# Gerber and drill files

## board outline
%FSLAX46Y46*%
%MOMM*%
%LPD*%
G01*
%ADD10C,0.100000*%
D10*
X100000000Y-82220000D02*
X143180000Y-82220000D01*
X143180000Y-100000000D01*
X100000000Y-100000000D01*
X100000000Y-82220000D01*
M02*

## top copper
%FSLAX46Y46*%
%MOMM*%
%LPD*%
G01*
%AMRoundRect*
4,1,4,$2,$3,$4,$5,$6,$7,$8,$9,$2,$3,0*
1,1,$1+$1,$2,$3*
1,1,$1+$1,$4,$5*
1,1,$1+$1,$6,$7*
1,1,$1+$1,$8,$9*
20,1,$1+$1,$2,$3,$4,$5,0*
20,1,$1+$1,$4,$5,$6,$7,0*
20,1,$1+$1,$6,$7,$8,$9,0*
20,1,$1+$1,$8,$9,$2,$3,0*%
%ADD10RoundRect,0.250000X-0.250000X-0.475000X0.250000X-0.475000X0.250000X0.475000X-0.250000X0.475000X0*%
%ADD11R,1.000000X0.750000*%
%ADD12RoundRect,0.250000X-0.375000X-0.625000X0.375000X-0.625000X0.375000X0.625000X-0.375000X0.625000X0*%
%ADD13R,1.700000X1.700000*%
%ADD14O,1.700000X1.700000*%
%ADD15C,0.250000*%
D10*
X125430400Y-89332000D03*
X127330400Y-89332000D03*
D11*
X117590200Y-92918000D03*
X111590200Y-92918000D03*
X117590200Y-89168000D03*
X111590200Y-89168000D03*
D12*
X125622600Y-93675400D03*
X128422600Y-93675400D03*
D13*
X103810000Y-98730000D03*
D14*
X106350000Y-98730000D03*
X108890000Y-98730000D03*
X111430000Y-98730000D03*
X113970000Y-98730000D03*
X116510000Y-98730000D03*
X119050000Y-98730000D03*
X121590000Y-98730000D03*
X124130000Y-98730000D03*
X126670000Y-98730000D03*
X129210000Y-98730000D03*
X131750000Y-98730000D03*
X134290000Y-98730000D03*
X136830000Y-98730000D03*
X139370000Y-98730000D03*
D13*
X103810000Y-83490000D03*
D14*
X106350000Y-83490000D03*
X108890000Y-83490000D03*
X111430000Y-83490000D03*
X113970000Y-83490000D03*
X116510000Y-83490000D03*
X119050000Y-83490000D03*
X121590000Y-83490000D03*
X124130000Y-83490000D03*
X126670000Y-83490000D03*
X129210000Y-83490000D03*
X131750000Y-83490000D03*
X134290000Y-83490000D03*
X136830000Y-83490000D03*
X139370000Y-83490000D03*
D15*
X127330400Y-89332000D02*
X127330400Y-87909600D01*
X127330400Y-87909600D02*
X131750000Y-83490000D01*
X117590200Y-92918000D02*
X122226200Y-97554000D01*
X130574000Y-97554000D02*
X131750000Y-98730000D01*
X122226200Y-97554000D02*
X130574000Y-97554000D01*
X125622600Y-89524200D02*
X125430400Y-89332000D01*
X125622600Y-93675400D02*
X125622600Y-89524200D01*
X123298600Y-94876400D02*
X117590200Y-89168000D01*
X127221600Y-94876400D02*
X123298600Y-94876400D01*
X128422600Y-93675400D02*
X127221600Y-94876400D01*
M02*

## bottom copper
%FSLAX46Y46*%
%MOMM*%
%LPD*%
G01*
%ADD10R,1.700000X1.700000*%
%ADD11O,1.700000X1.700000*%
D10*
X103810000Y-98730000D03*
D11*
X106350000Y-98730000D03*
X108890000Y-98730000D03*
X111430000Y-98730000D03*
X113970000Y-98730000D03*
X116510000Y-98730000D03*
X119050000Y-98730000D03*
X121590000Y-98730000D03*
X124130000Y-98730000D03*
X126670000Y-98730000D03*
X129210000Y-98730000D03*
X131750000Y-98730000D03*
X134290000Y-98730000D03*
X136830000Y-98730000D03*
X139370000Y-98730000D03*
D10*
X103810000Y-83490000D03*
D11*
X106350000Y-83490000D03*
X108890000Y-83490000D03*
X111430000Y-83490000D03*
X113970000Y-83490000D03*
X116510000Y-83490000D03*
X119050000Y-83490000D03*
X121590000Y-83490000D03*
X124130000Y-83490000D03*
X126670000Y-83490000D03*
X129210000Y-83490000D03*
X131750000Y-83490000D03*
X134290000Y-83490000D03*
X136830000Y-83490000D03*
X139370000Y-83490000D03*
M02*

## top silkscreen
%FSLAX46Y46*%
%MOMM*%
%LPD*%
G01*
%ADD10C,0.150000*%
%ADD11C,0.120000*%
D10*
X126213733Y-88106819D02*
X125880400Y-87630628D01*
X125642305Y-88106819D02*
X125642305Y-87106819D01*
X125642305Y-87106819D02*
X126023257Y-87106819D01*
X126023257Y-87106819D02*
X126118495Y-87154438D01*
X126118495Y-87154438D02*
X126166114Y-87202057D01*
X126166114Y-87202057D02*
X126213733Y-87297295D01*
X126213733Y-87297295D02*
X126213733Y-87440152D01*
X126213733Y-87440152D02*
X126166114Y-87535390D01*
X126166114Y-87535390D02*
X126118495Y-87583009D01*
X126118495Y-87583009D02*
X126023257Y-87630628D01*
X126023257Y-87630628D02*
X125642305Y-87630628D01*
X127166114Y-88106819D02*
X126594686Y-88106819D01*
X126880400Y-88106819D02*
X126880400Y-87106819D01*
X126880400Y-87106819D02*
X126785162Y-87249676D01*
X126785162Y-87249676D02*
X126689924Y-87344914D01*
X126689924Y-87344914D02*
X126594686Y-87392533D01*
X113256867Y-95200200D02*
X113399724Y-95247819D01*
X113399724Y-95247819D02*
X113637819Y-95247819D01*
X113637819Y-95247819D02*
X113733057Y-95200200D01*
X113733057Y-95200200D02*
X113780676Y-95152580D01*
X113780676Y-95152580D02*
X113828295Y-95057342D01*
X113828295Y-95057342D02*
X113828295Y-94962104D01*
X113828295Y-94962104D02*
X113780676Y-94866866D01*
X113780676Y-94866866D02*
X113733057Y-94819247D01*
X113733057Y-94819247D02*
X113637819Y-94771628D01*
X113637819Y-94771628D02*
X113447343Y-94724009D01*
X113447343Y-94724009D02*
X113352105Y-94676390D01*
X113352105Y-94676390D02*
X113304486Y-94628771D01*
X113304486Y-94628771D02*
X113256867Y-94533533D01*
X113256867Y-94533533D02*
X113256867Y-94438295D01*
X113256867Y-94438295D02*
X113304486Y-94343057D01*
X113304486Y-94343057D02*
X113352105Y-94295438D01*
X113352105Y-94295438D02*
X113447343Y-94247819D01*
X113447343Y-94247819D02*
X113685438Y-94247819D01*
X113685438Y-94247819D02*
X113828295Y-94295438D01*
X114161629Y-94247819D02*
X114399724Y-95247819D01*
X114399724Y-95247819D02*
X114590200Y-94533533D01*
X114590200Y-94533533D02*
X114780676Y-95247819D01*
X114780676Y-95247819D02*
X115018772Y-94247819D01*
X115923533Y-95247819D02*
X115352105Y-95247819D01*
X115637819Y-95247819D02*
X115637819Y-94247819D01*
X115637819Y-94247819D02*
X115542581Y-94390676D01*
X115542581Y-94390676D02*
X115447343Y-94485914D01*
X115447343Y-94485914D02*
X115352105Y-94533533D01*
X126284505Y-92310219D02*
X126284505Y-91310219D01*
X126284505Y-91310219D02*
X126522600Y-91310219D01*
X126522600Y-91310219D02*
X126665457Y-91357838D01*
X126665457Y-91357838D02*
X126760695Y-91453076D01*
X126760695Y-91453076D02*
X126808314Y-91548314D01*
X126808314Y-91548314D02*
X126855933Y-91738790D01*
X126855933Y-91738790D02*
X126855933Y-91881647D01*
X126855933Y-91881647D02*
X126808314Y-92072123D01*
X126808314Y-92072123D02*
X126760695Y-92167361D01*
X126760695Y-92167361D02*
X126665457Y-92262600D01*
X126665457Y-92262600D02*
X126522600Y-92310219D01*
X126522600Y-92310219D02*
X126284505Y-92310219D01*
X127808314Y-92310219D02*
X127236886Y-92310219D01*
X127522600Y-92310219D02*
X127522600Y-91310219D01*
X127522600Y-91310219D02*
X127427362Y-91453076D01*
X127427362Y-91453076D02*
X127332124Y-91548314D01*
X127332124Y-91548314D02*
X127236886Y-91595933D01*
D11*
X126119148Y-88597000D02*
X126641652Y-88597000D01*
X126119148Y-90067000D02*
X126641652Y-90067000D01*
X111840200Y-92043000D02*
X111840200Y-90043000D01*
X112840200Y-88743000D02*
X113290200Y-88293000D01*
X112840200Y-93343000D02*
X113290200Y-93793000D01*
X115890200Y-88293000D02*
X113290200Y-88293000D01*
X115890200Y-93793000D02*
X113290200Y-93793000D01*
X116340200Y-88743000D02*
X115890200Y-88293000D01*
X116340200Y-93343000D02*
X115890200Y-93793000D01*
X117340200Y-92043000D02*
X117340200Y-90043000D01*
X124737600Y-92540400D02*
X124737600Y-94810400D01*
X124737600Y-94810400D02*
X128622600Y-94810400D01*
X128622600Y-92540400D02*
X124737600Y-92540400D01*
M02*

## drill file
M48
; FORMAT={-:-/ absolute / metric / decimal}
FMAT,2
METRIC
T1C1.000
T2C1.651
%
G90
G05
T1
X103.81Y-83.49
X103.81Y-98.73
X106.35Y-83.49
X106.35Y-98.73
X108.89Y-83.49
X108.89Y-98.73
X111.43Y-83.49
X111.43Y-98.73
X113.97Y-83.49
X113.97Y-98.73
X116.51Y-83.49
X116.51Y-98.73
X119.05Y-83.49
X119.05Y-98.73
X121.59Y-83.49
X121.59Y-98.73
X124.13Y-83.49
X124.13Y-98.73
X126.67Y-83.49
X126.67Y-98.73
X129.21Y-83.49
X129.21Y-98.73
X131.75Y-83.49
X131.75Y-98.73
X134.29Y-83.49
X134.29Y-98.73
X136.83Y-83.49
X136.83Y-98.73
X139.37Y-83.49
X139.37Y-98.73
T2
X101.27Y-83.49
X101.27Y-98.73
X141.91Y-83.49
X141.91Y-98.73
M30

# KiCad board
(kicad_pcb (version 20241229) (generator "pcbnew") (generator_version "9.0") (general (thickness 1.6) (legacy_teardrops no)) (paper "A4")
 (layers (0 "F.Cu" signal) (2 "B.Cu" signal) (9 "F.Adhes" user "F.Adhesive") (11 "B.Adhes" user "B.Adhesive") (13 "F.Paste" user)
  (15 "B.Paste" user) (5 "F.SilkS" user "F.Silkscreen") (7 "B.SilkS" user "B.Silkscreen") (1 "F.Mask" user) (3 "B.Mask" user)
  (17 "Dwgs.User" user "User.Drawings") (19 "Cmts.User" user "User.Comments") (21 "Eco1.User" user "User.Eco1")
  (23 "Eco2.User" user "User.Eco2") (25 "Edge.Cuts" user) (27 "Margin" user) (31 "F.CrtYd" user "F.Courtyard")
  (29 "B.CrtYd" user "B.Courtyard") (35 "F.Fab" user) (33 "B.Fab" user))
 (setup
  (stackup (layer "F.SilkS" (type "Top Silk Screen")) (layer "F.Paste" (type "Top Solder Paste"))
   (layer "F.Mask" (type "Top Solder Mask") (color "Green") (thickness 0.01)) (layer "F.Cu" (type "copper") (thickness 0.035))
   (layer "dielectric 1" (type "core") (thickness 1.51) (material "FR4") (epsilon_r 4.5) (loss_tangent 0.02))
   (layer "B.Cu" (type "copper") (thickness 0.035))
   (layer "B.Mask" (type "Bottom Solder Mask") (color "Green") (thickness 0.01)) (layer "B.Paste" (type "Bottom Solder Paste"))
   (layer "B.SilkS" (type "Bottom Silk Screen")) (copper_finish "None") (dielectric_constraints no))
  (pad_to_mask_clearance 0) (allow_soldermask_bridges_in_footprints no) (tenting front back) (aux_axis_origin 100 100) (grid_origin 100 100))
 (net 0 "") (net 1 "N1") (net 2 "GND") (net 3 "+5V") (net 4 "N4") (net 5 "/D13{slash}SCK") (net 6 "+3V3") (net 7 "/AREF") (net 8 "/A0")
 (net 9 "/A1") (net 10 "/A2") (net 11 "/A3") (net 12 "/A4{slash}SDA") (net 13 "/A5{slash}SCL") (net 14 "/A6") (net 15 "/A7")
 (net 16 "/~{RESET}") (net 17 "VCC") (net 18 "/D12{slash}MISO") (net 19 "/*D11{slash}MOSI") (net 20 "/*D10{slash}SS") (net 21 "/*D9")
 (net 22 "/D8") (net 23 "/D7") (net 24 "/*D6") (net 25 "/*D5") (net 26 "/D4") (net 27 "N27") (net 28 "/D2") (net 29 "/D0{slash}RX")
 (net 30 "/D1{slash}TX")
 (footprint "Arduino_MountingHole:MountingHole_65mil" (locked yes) (layer "F.Cu") (at 101.27 83.49)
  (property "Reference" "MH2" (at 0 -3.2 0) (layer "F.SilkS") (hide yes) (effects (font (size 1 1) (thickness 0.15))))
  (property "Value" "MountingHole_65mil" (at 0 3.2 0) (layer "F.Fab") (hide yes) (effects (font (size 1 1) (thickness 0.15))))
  (pad "" np_thru_hole circle (at 0 0) (size 1.651 1.651) (drill 1.651) (layers "*.Cu" "*.Mask")))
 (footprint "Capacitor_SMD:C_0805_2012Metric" (layer "F.Cu") (at 126.3804 89.332)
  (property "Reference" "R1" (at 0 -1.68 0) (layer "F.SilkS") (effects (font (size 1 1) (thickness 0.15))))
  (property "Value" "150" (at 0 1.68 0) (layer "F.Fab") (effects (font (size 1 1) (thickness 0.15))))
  (fp_line (start -0.261252 -0.735) (end 0.261252 -0.735) (stroke (width 0.12) (type solid)) (layer "F.SilkS"))
  (fp_line (start -0.261252 0.735) (end 0.261252 0.735) (stroke (width 0.12) (type solid)) (layer "F.SilkS"))
  (pad "1" smd roundrect (at -0.95 0) (size 1 1.45) (layers "F.Cu" "F.Mask" "F.Paste") (roundrect_rratio 0.25) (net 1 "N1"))
  (pad "2" smd roundrect (at 0.95 0) (size 1 1.45) (layers "F.Cu" "F.Mask" "F.Paste") (roundrect_rratio 0.25) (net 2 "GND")))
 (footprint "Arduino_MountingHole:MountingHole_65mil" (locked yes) (layer "F.Cu") (at 141.91 98.73)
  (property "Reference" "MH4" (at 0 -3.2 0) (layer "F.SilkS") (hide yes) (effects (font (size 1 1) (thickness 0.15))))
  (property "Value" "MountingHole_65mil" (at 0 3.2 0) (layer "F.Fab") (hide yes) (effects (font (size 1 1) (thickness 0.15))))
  (pad "" np_thru_hole circle (at 0 0) (size 1.651 1.651) (drill 1.651) (layers "*.Cu" "*.Mask")))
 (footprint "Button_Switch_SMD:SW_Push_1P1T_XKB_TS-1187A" (layer "F.Cu") (at 114.5902 91.043 180)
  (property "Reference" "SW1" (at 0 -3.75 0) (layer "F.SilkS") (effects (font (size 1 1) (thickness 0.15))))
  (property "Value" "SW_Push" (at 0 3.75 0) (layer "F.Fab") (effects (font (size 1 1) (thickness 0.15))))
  (fp_line (start 2.75 -1) (end 2.75 1) (stroke (width 0.12) (type solid)) (layer "F.SilkS"))
  (fp_line (start 1.75 2.3) (end 1.3 2.75) (stroke (width 0.12) (type solid)) (layer "F.SilkS"))
  (fp_line (start 1.75 -2.3) (end 1.3 -2.75) (stroke (width 0.12) (type solid)) (layer "F.SilkS"))
  (fp_line (start -1.3 2.75) (end 1.3 2.75) (stroke (width 0.12) (type solid)) (layer "F.SilkS"))
  (fp_line (start -1.3 -2.75) (end 1.3 -2.75) (stroke (width 0.12) (type solid)) (layer "F.SilkS"))
  (fp_line (start -1.75 2.3) (end -1.3 2.75) (stroke (width 0.12) (type solid)) (layer "F.SilkS"))
  (fp_line (start -1.75 -2.3) (end -1.3 -2.75) (stroke (width 0.12) (type solid)) (layer "F.SilkS"))
  (fp_line (start -2.75 -1) (end -2.75 1) (stroke (width 0.12) (type solid)) (layer "F.SilkS"))
  (pad "1" smd rect (at -3 -1.875 180) (size 1 0.75) (layers "F.Cu" "F.Mask" "F.Paste") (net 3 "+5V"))
  (pad "1" smd rect (at 3 -1.875 180) (size 1 0.75) (layers "F.Cu" "F.Mask" "F.Paste") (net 3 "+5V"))
  (pad "2" smd rect (at -3 1.875 180) (size 1 0.75) (layers "F.Cu" "F.Mask" "F.Paste") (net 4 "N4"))
  (pad "2" smd rect (at 3 1.875 180) (size 1 0.75) (layers "F.Cu" "F.Mask" "F.Paste") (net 4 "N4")))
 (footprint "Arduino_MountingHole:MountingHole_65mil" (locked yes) (layer "F.Cu") (at 101.27 98.73)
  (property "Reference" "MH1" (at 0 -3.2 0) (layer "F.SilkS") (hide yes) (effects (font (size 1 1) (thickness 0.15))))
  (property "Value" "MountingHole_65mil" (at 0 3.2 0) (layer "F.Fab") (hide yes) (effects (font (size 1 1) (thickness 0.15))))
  (pad "" np_thru_hole circle (at 0 0) (size 1.651 1.651) (drill 1.651) (layers "*.Cu" "*.Mask")))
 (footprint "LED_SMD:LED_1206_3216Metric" (layer "F.Cu") (at 127.0226 93.6754)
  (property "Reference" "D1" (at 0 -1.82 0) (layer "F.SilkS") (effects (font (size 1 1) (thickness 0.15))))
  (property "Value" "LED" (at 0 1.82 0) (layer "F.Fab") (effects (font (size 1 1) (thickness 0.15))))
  (fp_line (start -2.285 -1.135) (end -2.285 1.135) (stroke (width 0.12) (type solid)) (layer "F.SilkS"))
  (fp_line (start -2.285 1.135) (end 1.6 1.135) (stroke (width 0.12) (type solid)) (layer "F.SilkS"))
  (fp_line (start 1.6 -1.135) (end -2.285 -1.135) (stroke (width 0.12) (type solid)) (layer "F.SilkS"))
  (pad "1" smd roundrect (at -1.4 0) (size 1.25 1.75) (layers "F.Cu" "F.Mask" "F.Paste") (roundrect_rratio 0.2) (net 1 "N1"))
  (pad "2" smd roundrect (at 1.4 0) (size 1.25 1.75) (layers "F.Cu" "F.Mask" "F.Paste") (roundrect_rratio 0.2) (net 4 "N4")))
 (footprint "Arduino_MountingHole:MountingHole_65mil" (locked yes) (layer "F.Cu") (at 141.91 83.49)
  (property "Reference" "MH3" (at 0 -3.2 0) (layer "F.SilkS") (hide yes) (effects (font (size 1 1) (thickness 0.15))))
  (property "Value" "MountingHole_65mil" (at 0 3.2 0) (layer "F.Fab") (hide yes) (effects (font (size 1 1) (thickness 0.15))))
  (pad "" np_thru_hole circle (at 0 0) (size 1.651 1.651) (drill 1.651) (layers "*.Cu" "*.Mask")))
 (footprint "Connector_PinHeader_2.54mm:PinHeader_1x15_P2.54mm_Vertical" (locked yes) (layer "B.Cu") (at 103.81 98.73 -90)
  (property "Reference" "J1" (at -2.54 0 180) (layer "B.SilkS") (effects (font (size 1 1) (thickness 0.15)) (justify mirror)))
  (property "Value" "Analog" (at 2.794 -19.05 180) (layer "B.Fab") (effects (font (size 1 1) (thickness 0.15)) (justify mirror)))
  (pad "1" thru_hole rect (at 0 0 270) (size 1.7 1.7) (drill 1) (layers "*.Cu" "*.Mask") (remove_unused_layers no) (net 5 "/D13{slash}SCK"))
  (pad "2" thru_hole oval (at 0 -2.54 270) (size 1.7 1.7) (drill 1) (layers "*.Cu" "*.Mask") (remove_unused_layers no) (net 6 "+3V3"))
  (pad "3" thru_hole oval (at 0 -5.08 270) (size 1.7 1.7) (drill 1) (layers "*.Cu" "*.Mask") (remove_unused_layers no) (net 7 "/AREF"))
  (pad "4" thru_hole oval (at 0 -7.62 270) (size 1.7 1.7) (drill 1) (layers "*.Cu" "*.Mask") (remove_unused_layers no) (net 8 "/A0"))
  (pad "5" thru_hole oval (at 0 -10.16 270) (size 1.7 1.7) (drill 1) (layers "*.Cu" "*.Mask") (remove_unused_layers no) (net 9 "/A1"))
  (pad "6" thru_hole oval (at 0 -12.7 270) (size 1.7 1.7) (drill 1) (layers "*.Cu" "*.Mask") (remove_unused_layers no) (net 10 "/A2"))
  (pad "7" thru_hole oval (at 0 -15.24 270) (size 1.7 1.7) (drill 1) (layers "*.Cu" "*.Mask") (remove_unused_layers no) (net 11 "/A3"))
  (pad "8" thru_hole oval (at 0 -17.78 270) (size 1.7 1.7) (drill 1) (layers "*.Cu" "*.Mask") (remove_unused_layers no)
   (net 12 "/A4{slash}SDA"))
  (pad "9" thru_hole oval (at 0 -20.32 270) (size 1.7 1.7) (drill 1) (layers "*.Cu" "*.Mask") (remove_unused_layers no)
   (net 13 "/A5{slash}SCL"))
  (pad "10" thru_hole oval (at 0 -22.86 270) (size 1.7 1.7) (drill 1) (layers "*.Cu" "*.Mask") (remove_unused_layers no) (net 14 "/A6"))
  (pad "11" thru_hole oval (at 0 -25.4 270) (size 1.7 1.7) (drill 1) (layers "*.Cu" "*.Mask") (remove_unused_layers no) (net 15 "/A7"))
  (pad "12" thru_hole oval (at 0 -27.94 270) (size 1.7 1.7) (drill 1) (layers "*.Cu" "*.Mask") (remove_unused_layers no) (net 3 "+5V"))
  (pad "13" thru_hole oval (at 0 -30.48 270) (size 1.7 1.7) (drill 1) (layers "*.Cu" "*.Mask") (remove_unused_layers no)
   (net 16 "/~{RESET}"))
  (pad "14" thru_hole oval (at 0 -33.02 270) (size 1.7 1.7) (drill 1) (layers "*.Cu" "*.Mask") (remove_unused_layers no) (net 2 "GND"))
  (pad "15" thru_hole oval (at 0 -35.56 270) (size 1.7 1.7) (drill 1) (layers "*.Cu" "*.Mask") (remove_unused_layers no) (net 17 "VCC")))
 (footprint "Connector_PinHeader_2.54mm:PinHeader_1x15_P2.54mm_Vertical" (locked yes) (layer "B.Cu") (at 103.81 83.49 -90)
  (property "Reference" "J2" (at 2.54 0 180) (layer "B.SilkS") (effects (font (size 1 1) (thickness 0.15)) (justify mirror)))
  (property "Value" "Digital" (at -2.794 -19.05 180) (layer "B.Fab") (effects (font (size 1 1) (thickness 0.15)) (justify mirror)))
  (pad "1" thru_hole rect (at 0 0 270) (size 1.7 1.7) (drill 1) (layers "*.Cu" "*.Mask") (remove_unused_layers no)
   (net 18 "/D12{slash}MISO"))
  (pad "2" thru_hole oval (at 0 -2.54 270) (size 1.7 1.7) (drill 1) (layers "*.Cu" "*.Mask") (remove_unused_layers no)
   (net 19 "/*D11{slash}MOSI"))
  (pad "3" thru_hole oval (at 0 -5.08 270) (size 1.7 1.7) (drill 1) (layers "*.Cu" "*.Mask") (remove_unused_layers no)
   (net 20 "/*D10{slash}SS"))
  (pad "4" thru_hole oval (at 0 -7.62 270) (size 1.7 1.7) (drill 1) (layers "*.Cu" "*.Mask") (remove_unused_layers no) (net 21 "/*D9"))
  (pad "5" thru_hole oval (at 0 -10.16 270) (size 1.7 1.7) (drill 1) (layers "*.Cu" "*.Mask") (remove_unused_layers no) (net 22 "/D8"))
  (pad "6" thru_hole oval (at 0 -12.7 270) (size 1.7 1.7) (drill 1) (layers "*.Cu" "*.Mask") (remove_unused_layers no) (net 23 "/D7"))
  (pad "7" thru_hole oval (at 0 -15.24 270) (size 1.7 1.7) (drill 1) (layers "*.Cu" "*.Mask") (remove_unused_layers no) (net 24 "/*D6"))
  (pad "8" thru_hole oval (at 0 -17.78 270) (size 1.7 1.7) (drill 1) (layers "*.Cu" "*.Mask") (remove_unused_layers no) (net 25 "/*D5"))
  (pad "9" thru_hole oval (at 0 -20.32 270) (size 1.7 1.7) (drill 1) (layers "*.Cu" "*.Mask") (remove_unused_layers no) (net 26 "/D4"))
  (pad "10" thru_hole oval (at 0 -22.86 270) (size 1.7 1.7) (drill 1) (layers "*.Cu" "*.Mask") (remove_unused_layers no) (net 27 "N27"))
  (pad "11" thru_hole oval (at 0 -25.4 270) (size 1.7 1.7) (drill 1) (layers "*.Cu" "*.Mask") (remove_unused_layers no) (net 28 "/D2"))
  (pad "12" thru_hole oval (at 0 -27.94 270) (size 1.7 1.7) (drill 1) (layers "*.Cu" "*.Mask") (remove_unused_layers no) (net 2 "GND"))
  (pad "13" thru_hole oval (at 0 -30.48 270) (size 1.7 1.7) (drill 1) (layers "*.Cu" "*.Mask") (remove_unused_layers no)
   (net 16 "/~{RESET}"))
  (pad "14" thru_hole oval (at 0 -33.02 270) (size 1.7 1.7) (drill 1) (layers "*.Cu" "*.Mask") (remove_unused_layers no)
   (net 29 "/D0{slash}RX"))
  (pad "15" thru_hole oval (at 0 -35.56 270) (size 1.7 1.7) (drill 1) (layers "*.Cu" "*.Mask") (remove_unused_layers no)
   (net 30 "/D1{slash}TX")))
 (gr_rect (start 100 82.22) (end 143.18 100) (stroke (width 0.1) (type solid)) (fill no) (layer "Edge.Cuts"))
 (segment (start 127.3304 89.332) (end 127.3304 87.9096) (width 0.25) (layer "F.Cu") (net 2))
 (segment (start 127.3304 87.9096) (end 131.75 83.49) (width 0.25) (layer "F.Cu") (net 2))
 (segment (start 117.5902 92.918) (end 122.2262 97.554) (width 0.25) (layer "F.Cu") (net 3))
 (segment (start 130.574 97.554) (end 131.75 98.73) (width 0.25) (layer "F.Cu") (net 3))
 (segment (start 122.2262 97.554) (end 130.574 97.554) (width 0.25) (layer "F.Cu") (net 3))
 (segment (start 125.6226 89.5242) (end 125.4304 89.332) (width 0.25) (layer "F.Cu") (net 1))
 (segment (start 125.6226 93.6754) (end 125.6226 89.5242) (width 0.25) (layer "F.Cu") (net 1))
 (segment (start 123.2986 94.8764) (end 117.5902 89.168) (width 0.25) (layer "F.Cu") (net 4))
 (segment (start 127.2216 94.8764) (end 123.2986 94.8764) (width 0.25) (layer "F.Cu") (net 4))
 (segment (start 128.4226 93.6754) (end 127.2216 94.8764) (width 0.25) (layer "F.Cu") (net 4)))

